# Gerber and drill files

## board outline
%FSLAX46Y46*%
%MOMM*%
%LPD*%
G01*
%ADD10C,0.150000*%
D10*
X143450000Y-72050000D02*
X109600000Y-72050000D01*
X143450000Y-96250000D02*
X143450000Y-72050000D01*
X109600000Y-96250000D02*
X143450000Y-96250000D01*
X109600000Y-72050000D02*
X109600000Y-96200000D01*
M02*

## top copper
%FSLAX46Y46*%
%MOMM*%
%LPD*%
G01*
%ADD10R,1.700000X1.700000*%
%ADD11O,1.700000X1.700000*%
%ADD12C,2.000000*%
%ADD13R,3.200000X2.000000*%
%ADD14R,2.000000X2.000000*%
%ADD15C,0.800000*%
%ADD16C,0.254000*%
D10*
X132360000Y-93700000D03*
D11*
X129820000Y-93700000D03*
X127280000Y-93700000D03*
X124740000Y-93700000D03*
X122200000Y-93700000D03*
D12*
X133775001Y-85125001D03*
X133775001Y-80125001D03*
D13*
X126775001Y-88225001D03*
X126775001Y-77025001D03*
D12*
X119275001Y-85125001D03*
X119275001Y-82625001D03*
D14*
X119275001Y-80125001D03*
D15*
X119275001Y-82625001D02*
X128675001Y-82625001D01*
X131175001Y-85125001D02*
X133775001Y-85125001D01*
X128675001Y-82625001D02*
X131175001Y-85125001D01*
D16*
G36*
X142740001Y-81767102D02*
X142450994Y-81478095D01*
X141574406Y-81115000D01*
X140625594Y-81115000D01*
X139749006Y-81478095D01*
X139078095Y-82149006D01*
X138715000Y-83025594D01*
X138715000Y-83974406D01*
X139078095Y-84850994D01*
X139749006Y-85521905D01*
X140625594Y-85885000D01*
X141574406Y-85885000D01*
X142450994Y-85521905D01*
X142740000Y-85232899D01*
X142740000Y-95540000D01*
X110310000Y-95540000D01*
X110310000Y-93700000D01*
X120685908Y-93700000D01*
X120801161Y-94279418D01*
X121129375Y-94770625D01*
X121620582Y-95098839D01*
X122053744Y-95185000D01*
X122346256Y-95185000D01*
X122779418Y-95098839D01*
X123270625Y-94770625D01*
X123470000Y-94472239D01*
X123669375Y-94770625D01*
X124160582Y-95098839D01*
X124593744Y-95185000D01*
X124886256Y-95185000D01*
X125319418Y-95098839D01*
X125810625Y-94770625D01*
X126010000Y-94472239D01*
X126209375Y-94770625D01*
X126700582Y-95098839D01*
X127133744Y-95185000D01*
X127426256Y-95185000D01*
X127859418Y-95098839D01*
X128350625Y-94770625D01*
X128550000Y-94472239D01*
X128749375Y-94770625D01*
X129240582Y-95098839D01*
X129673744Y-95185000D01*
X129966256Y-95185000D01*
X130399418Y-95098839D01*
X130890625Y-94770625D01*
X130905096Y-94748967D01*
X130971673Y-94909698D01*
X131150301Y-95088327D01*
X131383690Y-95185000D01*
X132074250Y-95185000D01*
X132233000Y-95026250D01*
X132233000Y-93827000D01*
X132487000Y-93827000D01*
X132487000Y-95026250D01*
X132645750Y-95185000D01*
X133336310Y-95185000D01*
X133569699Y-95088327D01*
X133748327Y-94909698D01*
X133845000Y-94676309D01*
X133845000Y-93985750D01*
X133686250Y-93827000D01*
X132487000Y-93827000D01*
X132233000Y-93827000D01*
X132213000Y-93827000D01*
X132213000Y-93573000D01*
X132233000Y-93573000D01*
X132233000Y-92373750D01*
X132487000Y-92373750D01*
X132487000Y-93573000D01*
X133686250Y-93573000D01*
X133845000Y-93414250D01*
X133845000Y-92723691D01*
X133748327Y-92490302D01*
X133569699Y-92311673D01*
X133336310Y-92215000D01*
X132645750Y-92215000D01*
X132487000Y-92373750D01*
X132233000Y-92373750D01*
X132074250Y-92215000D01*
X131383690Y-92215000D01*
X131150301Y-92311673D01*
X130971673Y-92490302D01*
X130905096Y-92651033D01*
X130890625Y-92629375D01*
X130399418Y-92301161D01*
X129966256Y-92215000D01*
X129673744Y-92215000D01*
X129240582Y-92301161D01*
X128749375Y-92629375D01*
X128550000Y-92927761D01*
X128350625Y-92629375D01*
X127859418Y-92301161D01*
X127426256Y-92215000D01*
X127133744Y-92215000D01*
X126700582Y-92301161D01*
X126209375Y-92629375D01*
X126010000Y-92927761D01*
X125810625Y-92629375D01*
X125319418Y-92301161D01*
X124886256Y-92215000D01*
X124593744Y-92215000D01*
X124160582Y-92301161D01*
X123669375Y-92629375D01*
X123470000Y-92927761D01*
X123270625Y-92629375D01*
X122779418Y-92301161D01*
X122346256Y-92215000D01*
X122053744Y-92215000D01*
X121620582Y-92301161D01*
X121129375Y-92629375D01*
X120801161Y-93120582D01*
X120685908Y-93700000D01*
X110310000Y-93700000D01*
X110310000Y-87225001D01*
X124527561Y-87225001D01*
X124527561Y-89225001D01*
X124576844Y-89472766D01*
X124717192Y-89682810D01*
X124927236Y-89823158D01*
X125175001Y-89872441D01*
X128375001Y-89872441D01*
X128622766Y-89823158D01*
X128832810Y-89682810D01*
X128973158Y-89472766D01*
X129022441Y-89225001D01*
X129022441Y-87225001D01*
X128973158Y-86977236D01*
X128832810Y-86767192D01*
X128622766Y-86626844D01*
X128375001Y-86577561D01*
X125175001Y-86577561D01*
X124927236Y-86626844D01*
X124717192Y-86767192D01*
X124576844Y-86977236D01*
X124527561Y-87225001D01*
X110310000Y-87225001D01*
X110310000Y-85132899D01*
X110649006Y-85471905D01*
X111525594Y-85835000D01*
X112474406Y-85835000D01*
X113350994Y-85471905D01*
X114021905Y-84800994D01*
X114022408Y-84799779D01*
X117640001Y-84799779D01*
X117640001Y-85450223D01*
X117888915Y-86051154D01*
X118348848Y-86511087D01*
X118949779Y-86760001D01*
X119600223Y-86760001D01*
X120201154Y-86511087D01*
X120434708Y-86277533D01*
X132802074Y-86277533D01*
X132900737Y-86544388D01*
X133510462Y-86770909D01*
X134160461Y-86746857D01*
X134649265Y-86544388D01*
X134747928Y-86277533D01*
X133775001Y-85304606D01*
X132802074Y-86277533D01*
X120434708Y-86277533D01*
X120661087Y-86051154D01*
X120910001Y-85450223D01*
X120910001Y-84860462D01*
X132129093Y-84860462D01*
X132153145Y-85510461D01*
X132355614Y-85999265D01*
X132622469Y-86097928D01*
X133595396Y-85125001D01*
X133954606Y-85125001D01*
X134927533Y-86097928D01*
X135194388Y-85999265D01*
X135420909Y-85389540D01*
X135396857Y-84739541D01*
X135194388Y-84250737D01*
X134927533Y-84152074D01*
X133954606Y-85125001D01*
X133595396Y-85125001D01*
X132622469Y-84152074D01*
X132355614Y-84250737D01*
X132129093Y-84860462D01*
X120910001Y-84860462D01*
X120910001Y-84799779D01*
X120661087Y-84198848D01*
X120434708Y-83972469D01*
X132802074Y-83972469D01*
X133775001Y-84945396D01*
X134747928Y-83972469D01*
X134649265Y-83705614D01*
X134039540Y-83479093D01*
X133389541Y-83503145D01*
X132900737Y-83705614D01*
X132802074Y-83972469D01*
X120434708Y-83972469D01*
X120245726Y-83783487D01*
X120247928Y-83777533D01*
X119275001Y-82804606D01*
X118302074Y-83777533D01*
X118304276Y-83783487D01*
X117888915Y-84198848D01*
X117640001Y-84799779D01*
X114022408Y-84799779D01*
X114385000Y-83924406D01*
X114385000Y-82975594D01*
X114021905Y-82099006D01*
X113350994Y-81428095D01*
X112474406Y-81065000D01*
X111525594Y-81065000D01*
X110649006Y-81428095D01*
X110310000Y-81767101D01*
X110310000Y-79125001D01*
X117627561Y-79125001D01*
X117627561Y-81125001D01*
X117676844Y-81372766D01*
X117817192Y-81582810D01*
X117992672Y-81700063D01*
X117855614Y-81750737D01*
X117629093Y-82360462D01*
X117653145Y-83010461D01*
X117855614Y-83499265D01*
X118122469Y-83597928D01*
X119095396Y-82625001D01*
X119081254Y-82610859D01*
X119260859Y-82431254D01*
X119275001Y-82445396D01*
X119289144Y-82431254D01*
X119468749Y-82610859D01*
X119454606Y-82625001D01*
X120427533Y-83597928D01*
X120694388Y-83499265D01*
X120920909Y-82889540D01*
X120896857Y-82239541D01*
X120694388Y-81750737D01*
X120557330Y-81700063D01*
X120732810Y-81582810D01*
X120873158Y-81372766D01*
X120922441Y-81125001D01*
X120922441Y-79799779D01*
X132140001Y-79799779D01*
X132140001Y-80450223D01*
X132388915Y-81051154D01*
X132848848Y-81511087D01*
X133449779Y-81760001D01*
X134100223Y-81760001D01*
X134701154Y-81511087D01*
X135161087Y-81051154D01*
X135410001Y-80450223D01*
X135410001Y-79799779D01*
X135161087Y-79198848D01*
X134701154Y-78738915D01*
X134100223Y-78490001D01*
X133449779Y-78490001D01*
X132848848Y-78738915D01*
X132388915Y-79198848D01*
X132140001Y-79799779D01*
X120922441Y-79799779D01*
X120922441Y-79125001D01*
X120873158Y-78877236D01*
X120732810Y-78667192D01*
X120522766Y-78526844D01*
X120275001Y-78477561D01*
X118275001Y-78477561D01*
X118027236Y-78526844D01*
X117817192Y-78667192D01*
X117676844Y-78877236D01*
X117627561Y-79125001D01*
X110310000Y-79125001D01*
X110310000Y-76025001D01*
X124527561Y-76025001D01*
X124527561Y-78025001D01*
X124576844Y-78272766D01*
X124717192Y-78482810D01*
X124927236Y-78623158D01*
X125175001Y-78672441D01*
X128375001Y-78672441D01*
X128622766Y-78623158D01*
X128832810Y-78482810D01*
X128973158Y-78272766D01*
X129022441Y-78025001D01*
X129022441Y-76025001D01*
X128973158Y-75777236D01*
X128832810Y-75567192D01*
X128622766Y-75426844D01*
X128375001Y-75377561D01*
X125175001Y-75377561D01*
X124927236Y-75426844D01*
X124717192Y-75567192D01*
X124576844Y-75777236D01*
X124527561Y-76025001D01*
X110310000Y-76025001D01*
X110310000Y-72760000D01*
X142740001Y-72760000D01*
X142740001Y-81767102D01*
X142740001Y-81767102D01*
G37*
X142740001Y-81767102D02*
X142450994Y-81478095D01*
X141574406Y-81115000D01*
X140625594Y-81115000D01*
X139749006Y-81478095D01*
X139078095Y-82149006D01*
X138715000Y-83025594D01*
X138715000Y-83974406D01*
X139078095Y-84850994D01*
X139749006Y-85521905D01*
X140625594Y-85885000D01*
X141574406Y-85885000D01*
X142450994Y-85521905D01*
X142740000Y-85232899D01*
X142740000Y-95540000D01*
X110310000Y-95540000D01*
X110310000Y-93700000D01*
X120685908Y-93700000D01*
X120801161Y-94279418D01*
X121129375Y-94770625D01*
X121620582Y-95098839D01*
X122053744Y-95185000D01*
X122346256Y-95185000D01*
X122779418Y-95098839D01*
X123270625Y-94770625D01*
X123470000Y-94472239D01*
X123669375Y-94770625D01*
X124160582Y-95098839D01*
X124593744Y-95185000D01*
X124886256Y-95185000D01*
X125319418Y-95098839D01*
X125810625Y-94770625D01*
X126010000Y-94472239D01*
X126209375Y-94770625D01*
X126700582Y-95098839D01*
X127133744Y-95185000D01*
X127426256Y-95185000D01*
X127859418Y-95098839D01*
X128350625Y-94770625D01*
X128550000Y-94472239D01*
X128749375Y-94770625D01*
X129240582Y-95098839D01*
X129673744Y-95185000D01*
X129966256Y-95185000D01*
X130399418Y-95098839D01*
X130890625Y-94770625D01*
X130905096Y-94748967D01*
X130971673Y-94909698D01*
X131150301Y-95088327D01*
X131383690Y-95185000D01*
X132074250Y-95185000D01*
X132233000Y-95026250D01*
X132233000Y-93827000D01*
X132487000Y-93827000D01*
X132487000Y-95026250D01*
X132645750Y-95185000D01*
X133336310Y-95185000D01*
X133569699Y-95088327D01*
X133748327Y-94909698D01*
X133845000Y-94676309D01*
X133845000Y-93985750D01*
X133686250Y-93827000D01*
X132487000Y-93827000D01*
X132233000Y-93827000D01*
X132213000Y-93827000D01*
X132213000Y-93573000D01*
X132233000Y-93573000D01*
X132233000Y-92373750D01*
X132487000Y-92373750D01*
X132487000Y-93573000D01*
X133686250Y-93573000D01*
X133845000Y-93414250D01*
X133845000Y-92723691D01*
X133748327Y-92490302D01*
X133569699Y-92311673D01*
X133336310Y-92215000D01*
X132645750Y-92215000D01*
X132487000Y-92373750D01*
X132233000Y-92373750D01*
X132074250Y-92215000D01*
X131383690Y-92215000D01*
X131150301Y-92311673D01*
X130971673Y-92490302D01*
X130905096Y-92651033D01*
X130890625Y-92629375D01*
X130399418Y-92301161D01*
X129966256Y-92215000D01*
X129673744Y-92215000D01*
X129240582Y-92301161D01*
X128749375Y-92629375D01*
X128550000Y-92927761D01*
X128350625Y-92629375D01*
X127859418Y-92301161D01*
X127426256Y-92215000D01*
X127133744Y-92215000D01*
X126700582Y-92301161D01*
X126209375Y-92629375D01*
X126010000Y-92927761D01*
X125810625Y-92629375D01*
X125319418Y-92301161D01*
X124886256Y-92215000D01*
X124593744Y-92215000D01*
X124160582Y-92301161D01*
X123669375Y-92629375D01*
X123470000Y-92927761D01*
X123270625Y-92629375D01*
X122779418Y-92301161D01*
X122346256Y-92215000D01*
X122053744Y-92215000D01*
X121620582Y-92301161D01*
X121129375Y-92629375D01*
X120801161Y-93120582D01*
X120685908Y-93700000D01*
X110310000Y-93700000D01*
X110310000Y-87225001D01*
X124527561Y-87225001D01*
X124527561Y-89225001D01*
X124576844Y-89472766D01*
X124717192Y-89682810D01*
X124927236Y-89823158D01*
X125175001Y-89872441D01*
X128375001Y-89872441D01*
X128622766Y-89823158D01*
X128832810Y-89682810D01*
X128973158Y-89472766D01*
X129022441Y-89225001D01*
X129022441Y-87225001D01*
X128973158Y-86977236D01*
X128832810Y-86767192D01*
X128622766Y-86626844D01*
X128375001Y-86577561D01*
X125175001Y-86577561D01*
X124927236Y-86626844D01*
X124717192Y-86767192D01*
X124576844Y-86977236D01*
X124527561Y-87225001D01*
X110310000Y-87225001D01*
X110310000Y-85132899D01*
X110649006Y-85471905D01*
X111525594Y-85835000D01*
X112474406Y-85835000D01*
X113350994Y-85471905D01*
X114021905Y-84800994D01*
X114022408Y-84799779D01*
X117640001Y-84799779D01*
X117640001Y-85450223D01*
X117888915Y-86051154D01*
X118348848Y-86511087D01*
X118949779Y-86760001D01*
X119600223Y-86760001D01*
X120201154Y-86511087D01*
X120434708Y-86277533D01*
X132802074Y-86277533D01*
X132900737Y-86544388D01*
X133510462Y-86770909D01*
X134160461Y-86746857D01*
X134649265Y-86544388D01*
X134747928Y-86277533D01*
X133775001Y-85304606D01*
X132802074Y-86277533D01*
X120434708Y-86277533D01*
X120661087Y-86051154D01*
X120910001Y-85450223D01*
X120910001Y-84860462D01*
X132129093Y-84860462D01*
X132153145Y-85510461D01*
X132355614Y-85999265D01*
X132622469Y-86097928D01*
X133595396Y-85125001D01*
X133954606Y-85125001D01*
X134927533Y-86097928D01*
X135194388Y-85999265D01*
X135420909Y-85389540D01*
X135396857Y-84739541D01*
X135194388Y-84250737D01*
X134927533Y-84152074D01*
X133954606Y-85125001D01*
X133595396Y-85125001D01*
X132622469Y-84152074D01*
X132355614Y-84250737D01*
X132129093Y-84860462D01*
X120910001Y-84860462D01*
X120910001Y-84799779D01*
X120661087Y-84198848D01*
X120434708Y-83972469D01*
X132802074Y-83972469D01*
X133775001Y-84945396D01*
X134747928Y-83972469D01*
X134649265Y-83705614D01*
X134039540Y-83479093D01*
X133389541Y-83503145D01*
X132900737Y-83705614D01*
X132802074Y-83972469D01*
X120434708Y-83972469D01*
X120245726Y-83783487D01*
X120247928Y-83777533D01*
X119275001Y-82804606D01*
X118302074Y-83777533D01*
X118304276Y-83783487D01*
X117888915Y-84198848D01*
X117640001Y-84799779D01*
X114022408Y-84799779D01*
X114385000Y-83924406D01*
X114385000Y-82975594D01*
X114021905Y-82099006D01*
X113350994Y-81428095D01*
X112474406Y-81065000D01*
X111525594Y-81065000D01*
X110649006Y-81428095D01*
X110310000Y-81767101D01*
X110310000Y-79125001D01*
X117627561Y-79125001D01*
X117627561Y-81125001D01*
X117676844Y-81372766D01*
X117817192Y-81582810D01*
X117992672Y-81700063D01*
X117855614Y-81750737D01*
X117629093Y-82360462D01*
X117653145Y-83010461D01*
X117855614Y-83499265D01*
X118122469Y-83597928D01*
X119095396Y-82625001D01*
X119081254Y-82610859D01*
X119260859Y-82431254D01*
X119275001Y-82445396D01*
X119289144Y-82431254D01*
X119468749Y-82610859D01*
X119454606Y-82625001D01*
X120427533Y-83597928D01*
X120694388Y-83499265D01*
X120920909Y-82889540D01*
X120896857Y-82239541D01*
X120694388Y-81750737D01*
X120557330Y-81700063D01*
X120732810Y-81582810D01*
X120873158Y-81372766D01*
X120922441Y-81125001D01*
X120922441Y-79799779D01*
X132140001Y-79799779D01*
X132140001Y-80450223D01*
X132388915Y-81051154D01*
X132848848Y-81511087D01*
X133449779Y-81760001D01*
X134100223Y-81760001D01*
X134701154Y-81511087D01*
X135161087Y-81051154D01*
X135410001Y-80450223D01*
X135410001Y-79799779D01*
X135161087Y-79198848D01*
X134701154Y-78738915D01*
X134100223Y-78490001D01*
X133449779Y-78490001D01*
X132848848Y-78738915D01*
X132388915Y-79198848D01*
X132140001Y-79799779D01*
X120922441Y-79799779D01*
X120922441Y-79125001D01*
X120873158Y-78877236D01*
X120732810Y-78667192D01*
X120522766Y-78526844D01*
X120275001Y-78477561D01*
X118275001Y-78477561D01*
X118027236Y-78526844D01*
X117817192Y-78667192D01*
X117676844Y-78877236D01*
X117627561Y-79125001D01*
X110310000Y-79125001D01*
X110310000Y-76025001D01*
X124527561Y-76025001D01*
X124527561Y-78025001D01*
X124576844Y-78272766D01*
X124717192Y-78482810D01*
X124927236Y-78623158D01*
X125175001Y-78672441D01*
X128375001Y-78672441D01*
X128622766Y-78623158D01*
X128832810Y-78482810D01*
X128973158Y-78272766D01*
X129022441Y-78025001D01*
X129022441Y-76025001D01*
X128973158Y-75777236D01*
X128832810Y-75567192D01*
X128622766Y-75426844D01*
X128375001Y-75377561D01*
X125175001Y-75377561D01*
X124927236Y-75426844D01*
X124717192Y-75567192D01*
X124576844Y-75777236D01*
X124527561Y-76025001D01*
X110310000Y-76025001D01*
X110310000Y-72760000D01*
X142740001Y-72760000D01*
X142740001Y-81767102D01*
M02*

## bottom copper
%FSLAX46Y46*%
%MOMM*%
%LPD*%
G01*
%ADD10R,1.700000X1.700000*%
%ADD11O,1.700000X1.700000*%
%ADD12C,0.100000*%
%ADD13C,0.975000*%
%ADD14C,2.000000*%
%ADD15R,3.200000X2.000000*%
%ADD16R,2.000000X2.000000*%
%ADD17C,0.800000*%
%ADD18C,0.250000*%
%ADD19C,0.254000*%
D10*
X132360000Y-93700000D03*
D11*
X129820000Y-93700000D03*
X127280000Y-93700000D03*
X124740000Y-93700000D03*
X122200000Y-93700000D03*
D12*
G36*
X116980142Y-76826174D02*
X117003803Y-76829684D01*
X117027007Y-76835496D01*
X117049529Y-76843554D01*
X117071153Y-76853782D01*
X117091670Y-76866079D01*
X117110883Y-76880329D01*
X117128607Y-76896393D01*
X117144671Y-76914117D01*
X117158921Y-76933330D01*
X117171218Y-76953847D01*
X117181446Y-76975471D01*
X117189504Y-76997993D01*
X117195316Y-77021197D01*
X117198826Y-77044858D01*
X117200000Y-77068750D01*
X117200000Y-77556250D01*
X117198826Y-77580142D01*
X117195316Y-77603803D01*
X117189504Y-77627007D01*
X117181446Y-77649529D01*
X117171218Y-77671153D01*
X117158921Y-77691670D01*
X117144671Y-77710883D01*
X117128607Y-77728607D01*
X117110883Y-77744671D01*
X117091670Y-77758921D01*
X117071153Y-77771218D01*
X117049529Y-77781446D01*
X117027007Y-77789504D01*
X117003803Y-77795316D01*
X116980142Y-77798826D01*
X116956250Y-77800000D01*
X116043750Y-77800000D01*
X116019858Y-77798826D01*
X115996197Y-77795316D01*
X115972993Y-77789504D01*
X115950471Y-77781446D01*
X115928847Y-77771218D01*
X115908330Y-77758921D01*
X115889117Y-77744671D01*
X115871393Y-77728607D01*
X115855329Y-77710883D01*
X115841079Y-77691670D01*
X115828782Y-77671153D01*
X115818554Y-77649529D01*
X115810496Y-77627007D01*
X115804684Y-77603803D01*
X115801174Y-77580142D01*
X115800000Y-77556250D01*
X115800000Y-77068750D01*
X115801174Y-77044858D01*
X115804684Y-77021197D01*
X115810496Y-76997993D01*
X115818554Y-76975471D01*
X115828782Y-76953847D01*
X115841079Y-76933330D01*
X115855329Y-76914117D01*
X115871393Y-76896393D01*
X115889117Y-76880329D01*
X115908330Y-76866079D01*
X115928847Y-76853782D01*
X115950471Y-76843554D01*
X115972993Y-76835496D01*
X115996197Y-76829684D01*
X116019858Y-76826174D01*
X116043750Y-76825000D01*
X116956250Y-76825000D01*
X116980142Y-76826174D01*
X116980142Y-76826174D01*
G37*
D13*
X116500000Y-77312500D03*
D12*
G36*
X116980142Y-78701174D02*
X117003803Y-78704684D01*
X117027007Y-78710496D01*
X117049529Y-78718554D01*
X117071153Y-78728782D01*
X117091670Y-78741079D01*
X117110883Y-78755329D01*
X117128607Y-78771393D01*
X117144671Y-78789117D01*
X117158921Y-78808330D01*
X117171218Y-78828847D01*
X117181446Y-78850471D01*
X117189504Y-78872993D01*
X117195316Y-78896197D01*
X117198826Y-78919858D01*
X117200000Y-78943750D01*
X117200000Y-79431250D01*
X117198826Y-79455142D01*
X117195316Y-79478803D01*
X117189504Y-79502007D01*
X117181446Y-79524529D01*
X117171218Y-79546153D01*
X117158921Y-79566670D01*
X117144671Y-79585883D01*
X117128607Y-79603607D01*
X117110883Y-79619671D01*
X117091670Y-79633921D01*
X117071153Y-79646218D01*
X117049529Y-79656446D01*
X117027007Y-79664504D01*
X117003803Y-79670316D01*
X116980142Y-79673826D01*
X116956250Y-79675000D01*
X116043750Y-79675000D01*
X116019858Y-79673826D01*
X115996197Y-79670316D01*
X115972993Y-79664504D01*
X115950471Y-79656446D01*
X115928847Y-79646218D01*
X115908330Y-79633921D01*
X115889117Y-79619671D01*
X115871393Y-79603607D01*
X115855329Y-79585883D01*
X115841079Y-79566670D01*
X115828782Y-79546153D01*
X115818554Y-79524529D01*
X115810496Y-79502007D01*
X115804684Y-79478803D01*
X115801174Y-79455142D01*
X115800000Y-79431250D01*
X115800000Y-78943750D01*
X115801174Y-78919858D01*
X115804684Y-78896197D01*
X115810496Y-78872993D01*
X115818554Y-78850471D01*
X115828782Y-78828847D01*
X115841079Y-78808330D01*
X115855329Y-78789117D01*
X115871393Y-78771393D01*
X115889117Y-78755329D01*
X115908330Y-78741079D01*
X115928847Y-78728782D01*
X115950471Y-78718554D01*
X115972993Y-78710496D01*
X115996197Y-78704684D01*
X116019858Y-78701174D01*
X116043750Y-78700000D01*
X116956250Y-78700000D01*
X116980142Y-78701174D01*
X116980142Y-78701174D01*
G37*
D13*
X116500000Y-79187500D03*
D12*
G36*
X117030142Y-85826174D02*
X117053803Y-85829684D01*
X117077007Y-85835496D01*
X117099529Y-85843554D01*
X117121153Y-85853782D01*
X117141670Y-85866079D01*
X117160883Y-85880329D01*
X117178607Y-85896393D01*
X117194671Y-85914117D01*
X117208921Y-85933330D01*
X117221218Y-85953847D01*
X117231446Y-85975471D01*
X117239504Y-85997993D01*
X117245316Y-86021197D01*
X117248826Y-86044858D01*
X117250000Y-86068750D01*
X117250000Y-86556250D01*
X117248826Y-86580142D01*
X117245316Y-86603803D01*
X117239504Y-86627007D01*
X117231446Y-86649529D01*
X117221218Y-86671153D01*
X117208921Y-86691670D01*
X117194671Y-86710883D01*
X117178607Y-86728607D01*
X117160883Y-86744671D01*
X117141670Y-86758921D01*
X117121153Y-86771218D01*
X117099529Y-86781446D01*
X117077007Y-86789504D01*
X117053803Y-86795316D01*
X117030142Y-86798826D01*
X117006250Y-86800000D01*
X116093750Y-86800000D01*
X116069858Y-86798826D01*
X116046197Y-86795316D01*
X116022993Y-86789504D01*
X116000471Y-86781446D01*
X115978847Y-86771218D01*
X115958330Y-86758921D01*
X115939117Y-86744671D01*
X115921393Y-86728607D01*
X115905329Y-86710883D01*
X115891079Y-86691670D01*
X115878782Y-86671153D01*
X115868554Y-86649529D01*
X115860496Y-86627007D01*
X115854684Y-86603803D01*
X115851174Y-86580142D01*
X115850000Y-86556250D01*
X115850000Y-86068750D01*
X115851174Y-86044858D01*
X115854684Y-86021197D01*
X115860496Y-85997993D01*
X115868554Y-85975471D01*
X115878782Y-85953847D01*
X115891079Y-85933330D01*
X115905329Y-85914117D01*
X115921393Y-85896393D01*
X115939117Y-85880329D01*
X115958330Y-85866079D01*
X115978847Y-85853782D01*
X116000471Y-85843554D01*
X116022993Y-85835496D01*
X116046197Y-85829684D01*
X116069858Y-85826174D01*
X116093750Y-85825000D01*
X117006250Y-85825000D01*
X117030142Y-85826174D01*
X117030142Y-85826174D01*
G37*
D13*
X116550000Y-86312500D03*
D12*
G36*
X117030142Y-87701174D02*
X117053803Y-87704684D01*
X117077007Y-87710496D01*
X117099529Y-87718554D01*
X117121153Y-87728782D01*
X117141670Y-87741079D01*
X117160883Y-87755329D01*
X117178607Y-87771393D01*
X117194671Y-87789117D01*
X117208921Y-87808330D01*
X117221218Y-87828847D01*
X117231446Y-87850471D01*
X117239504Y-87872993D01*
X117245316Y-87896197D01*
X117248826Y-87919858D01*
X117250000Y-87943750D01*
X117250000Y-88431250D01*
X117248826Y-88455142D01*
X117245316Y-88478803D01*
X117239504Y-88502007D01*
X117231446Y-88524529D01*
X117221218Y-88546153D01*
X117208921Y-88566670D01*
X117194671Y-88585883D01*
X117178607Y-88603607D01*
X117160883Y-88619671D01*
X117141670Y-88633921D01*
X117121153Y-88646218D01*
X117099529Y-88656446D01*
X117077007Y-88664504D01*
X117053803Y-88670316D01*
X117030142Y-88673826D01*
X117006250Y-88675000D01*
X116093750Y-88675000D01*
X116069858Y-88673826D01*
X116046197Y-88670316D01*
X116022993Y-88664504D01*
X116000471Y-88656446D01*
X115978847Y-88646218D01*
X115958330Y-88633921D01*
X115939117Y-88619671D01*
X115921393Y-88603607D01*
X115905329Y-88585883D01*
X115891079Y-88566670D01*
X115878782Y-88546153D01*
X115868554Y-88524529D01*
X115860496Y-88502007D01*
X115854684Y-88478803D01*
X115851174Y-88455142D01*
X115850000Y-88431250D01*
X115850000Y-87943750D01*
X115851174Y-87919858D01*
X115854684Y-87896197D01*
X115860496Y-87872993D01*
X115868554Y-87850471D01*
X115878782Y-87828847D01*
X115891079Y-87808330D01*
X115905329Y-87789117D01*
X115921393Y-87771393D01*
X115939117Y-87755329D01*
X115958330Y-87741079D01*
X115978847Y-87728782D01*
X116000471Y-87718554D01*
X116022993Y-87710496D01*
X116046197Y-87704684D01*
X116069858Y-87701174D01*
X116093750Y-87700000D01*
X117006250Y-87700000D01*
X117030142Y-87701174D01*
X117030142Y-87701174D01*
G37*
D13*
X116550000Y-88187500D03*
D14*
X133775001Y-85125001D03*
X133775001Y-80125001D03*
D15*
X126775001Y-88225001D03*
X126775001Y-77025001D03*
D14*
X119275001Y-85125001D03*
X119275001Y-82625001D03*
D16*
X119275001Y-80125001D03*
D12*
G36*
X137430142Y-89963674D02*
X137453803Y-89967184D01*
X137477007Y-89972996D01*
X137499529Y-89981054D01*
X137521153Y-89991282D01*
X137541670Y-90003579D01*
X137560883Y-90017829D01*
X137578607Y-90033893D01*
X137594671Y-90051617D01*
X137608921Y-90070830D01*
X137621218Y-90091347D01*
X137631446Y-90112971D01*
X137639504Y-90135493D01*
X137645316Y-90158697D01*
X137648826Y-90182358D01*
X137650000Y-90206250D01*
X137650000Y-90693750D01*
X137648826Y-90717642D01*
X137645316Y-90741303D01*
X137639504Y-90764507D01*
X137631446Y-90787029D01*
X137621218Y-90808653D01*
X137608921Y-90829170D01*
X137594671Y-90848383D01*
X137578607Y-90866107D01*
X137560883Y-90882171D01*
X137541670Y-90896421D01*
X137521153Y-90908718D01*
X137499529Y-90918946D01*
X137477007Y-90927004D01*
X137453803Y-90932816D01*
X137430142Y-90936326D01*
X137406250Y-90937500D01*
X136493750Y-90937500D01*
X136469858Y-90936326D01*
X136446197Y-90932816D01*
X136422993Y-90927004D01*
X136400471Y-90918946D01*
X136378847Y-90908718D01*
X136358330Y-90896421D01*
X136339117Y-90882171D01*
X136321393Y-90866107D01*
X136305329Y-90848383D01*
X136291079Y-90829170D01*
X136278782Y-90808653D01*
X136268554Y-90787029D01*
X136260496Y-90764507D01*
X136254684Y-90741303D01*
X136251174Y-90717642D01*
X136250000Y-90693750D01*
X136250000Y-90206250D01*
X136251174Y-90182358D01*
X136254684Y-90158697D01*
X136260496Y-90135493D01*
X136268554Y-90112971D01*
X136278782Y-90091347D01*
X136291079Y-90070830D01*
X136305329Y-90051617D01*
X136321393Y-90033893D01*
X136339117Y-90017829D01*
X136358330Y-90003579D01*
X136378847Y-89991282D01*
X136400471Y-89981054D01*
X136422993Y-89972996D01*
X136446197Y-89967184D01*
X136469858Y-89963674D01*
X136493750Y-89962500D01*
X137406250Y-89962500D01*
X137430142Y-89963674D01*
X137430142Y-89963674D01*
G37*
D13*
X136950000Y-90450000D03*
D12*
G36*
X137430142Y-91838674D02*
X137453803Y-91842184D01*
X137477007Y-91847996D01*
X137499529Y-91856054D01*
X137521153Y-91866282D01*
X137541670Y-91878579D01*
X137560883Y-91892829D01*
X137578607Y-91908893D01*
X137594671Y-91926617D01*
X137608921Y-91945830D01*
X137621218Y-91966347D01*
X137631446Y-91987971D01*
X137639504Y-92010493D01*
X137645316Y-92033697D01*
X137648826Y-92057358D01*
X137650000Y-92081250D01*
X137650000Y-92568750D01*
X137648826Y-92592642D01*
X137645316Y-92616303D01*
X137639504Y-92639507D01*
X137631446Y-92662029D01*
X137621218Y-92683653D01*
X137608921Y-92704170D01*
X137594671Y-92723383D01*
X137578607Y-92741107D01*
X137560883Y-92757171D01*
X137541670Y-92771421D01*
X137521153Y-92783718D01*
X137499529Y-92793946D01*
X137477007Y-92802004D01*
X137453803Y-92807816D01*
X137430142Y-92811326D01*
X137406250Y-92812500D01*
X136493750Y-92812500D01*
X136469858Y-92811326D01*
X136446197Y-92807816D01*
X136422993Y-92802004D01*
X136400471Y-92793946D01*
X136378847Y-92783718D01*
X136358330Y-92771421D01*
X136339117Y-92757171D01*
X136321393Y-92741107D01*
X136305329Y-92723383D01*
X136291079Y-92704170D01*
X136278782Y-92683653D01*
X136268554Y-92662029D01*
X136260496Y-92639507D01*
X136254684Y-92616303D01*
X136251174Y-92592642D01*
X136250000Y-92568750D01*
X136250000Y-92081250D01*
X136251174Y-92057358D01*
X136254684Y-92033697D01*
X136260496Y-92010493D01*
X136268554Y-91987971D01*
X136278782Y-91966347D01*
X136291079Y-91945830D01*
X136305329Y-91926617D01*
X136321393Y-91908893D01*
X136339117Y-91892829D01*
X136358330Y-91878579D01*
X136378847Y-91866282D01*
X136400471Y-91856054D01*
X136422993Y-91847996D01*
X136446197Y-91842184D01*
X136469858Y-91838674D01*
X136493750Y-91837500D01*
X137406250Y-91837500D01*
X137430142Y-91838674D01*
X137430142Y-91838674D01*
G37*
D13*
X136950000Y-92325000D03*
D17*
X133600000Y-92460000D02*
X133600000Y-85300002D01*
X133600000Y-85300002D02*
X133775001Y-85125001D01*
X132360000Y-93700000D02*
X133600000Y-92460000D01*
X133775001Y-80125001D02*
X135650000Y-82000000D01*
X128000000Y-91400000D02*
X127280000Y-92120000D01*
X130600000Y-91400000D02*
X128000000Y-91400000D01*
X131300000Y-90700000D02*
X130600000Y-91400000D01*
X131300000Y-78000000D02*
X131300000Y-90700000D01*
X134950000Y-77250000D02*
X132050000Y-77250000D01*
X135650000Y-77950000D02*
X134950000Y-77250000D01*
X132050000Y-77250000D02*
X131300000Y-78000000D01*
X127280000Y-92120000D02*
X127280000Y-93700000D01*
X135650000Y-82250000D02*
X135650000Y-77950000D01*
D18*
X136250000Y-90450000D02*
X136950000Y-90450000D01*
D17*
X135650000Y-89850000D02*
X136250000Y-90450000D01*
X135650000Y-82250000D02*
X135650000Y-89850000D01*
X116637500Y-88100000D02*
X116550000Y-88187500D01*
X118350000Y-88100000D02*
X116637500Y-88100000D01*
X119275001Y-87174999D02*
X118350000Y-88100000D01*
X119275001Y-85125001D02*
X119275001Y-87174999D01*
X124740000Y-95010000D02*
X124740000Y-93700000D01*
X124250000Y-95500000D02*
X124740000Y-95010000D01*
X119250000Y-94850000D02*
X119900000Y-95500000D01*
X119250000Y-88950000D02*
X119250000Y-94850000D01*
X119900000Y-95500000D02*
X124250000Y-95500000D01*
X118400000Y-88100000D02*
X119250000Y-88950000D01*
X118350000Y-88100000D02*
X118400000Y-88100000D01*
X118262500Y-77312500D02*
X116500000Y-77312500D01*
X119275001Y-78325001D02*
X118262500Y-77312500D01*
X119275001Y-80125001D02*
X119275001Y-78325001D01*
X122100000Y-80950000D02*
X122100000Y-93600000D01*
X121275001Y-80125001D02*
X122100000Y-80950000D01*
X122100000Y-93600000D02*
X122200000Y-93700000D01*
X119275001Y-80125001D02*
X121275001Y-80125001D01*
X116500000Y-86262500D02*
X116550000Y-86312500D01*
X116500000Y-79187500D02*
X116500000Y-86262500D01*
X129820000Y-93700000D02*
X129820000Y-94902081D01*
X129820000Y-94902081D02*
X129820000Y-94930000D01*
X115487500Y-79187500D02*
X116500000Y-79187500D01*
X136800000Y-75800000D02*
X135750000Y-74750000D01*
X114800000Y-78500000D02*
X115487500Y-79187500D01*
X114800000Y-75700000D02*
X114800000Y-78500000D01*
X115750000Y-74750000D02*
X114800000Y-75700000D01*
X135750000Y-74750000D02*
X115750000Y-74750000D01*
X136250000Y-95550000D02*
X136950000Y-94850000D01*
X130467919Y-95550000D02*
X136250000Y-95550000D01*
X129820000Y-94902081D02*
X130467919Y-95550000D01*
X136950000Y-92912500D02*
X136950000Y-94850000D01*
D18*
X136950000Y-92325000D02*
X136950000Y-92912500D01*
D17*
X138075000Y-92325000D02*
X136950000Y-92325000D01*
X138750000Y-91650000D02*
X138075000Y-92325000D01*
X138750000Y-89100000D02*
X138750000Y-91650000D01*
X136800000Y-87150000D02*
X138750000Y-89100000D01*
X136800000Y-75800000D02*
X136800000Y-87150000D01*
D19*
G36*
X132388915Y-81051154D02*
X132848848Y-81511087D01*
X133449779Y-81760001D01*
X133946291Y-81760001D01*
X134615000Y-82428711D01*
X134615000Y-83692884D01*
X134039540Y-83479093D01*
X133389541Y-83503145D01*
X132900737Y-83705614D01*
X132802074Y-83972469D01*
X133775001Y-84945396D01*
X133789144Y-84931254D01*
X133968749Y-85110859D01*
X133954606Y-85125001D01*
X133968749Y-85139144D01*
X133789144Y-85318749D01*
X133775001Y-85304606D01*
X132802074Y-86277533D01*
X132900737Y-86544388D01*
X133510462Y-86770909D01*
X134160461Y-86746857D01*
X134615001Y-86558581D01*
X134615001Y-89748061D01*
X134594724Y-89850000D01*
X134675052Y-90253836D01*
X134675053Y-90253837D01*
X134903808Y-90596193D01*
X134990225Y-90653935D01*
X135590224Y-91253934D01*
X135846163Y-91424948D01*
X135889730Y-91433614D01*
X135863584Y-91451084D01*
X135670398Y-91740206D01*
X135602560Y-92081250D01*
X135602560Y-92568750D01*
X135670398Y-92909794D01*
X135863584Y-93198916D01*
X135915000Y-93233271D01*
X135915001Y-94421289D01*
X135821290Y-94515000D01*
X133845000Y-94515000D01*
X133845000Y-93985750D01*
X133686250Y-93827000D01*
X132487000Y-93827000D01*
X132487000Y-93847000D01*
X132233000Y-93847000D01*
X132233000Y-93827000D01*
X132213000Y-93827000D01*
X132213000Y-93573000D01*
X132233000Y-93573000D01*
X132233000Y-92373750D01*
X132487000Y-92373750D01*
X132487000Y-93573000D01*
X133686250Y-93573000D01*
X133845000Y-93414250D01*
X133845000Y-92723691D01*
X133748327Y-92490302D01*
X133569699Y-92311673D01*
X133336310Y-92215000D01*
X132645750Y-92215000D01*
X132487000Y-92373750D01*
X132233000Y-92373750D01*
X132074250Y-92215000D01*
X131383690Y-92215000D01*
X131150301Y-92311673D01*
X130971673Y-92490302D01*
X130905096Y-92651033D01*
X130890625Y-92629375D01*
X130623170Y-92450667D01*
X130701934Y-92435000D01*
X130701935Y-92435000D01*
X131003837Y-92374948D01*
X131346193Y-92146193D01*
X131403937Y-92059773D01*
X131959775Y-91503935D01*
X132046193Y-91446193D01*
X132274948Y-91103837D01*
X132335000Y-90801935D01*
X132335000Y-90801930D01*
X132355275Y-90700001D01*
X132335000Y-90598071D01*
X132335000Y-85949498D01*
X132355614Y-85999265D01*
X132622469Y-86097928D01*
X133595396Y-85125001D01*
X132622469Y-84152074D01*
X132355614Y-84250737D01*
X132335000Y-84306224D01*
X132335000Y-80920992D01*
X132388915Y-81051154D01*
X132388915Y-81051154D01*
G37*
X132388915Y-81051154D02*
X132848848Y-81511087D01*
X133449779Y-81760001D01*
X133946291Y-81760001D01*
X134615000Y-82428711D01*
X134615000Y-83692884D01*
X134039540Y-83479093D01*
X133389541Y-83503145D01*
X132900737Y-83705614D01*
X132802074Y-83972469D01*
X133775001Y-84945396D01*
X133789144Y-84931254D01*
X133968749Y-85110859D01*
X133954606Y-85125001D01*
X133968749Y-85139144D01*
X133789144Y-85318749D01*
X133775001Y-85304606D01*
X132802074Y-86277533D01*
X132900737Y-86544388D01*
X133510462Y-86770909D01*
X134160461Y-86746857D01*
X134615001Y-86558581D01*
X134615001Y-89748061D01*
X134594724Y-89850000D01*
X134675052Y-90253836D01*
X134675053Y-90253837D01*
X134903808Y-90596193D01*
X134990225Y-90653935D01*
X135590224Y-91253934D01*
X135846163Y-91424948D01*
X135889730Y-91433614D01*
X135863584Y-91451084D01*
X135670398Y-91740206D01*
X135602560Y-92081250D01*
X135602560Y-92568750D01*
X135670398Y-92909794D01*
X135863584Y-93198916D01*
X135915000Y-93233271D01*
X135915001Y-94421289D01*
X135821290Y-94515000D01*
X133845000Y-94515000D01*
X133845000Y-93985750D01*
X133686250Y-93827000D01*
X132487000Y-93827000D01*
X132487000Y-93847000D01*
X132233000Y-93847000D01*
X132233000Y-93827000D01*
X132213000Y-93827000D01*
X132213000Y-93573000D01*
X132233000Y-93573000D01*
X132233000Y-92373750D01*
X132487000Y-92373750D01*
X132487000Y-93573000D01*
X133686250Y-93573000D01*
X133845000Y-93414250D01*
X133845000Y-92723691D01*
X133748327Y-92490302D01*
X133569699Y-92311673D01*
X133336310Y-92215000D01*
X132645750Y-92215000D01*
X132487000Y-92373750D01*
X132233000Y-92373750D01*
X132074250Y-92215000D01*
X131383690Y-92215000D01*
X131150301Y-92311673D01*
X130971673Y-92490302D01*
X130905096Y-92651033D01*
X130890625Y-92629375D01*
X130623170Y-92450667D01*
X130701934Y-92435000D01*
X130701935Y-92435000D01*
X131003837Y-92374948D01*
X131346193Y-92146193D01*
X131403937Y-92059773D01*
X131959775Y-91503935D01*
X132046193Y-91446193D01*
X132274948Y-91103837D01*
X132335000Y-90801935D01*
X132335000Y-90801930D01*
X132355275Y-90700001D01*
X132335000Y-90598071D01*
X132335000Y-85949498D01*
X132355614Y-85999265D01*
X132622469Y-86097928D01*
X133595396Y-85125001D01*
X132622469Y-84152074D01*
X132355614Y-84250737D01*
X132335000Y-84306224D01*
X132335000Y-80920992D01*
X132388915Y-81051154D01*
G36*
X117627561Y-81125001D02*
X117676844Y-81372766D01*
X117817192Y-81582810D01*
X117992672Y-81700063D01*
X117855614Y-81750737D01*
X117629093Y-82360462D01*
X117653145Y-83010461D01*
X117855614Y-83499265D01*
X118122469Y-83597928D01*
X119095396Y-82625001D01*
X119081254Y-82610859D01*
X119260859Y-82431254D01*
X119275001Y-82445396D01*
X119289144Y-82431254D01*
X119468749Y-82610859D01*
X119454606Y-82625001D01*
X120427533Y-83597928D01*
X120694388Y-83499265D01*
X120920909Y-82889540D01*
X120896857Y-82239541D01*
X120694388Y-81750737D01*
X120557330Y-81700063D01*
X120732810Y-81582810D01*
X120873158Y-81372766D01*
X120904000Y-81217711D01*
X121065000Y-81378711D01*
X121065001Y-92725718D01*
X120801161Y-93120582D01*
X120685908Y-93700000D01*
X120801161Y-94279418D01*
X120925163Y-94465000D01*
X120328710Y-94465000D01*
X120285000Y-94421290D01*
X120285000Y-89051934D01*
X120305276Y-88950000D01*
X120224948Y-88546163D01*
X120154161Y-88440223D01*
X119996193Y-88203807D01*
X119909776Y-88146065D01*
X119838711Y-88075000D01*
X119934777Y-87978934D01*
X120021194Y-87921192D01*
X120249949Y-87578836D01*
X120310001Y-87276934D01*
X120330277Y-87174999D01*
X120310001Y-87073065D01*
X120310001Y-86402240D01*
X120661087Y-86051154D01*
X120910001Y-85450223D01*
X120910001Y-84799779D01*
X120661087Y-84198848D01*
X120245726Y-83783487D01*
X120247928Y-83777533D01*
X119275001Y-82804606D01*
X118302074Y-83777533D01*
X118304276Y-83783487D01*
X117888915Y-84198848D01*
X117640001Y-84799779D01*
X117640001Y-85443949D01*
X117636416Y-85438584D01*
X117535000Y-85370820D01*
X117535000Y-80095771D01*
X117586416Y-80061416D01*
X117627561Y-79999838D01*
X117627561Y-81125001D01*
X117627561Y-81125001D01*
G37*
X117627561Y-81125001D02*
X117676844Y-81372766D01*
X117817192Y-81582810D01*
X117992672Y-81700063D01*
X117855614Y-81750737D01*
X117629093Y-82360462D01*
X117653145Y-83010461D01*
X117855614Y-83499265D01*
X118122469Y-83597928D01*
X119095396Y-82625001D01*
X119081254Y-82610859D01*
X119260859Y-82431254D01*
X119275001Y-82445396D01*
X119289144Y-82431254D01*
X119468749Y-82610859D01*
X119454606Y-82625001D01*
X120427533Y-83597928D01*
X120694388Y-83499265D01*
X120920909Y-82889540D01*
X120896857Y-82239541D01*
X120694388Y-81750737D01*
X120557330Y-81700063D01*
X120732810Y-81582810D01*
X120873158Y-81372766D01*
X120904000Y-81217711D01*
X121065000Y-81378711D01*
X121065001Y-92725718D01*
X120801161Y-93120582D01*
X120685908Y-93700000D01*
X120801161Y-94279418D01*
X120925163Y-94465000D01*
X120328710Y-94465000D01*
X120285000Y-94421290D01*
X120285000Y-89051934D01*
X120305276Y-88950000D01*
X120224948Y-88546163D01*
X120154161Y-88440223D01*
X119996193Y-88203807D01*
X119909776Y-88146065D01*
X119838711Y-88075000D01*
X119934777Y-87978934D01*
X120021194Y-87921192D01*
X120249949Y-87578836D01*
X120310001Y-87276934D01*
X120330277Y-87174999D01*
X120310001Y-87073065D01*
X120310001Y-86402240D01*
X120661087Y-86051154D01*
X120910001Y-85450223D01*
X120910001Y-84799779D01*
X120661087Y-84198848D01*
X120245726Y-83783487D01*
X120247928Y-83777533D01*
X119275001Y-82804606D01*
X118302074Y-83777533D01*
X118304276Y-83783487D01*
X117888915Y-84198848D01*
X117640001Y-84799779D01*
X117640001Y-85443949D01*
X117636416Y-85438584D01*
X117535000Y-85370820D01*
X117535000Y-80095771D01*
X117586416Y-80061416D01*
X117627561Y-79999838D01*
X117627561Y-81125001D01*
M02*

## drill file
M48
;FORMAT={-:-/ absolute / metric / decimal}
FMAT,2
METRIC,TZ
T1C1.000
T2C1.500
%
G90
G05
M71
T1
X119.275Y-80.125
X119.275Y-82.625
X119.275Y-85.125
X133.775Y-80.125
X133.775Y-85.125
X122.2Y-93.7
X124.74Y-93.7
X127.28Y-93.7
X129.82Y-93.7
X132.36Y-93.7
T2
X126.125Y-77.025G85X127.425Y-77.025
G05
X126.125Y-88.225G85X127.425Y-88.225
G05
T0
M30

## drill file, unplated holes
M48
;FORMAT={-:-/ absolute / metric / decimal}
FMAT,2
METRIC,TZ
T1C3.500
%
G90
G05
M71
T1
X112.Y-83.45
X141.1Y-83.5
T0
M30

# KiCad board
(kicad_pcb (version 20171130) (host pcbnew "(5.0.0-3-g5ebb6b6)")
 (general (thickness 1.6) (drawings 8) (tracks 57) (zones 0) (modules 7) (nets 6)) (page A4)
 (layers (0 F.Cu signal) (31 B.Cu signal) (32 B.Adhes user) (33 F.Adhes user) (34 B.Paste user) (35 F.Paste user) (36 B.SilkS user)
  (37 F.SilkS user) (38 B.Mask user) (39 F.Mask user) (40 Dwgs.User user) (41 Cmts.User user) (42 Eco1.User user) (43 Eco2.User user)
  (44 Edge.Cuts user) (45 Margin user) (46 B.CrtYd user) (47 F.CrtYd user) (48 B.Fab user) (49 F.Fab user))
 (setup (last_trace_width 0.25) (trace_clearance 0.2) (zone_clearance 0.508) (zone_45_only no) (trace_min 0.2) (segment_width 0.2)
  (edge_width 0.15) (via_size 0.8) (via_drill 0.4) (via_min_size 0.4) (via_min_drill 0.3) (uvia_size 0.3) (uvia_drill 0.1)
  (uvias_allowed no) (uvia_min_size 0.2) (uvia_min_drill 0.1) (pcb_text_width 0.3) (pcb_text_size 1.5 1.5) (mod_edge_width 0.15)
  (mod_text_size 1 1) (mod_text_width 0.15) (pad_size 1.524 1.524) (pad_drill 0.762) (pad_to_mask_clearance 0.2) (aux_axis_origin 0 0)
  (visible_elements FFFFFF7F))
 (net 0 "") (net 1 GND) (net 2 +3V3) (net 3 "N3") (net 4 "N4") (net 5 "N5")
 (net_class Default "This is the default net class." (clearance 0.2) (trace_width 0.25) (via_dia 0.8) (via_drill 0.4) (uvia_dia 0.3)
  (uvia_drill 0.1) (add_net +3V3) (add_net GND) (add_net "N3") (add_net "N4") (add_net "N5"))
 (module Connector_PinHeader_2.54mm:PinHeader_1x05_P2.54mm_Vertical (layer F.Cu) (at 132.36 93.7 270)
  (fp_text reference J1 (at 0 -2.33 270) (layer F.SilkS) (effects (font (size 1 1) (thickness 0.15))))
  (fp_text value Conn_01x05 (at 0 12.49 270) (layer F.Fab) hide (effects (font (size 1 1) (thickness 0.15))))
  (pad 1 thru_hole rect (at 0 0 270) (size 1.7 1.7) (drill 1) (layers *.Cu *.Mask) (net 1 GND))
  (pad 2 thru_hole oval (at 0 2.54 270) (size 1.7 1.7) (drill 1) (layers *.Cu *.Mask) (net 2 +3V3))
  (pad 3 thru_hole oval (at 0 5.08 270) (size 1.7 1.7) (drill 1) (layers *.Cu *.Mask) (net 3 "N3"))
  (pad 4 thru_hole oval (at 0 7.62 270) (size 1.7 1.7) (drill 1) (layers *.Cu *.Mask) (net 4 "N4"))
  (pad 5 thru_hole oval (at 0 10.16 270) (size 1.7 1.7) (drill 1) (layers *.Cu *.Mask) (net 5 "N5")))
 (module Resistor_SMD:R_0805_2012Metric (layer B.Cu) (at 116.5 78.25 270)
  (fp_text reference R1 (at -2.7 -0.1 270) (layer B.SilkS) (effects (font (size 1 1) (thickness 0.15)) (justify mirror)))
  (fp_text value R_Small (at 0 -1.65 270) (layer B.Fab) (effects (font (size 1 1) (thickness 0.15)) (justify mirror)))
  (pad 1 smd roundrect (at -0.9375 0 270) (size 0.975 1.4) (layers B.Cu B.Paste B.Mask) (roundrect_rratio 0.25) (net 5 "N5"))
  (pad 2 smd roundrect (at 0.9375 0 270) (size 0.975 1.4) (layers B.Cu B.Paste B.Mask) (roundrect_rratio 0.25) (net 2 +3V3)))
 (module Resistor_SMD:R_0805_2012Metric (layer B.Cu) (at 116.55 87.25 90)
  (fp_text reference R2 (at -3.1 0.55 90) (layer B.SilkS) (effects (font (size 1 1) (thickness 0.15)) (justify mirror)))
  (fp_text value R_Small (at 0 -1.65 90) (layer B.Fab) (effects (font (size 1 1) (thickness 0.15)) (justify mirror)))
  (pad 2 smd roundrect (at 0.9375 0 90) (size 0.975 1.4) (layers B.Cu B.Paste B.Mask) (roundrect_rratio 0.25) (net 2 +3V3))
  (pad 1 smd roundrect (at -0.9375 0 90) (size 0.975 1.4) (layers B.Cu B.Paste B.Mask) (roundrect_rratio 0.25) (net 4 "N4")))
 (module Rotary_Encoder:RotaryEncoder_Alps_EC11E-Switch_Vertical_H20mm (layer F.Cu) (at 119.275001 80.125001)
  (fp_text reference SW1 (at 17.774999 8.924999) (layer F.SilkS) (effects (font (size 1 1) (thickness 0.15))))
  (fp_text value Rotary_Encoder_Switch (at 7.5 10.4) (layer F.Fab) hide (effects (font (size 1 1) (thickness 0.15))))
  (pad S1 thru_hole circle (at 14.5 5) (size 2 2) (drill 1) (layers *.Cu *.Mask) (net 1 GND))
  (pad S2 thru_hole circle (at 14.5 0) (size 2 2) (drill 1) (layers *.Cu *.Mask) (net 3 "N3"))
  (pad MP thru_hole rect (at 7.5 8.1) (size 3.2 2) (drill oval 2.8 1.5) (layers *.Cu *.Mask))
  (pad MP thru_hole rect (at 7.5 -3.1) (size 3.2 2) (drill oval 2.8 1.5) (layers *.Cu *.Mask))
  (pad B thru_hole circle (at 0 5) (size 2 2) (drill 1) (layers *.Cu *.Mask) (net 4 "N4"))
  (pad C thru_hole circle (at 0 2.5) (size 2 2) (drill 1) (layers *.Cu *.Mask) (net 1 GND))
  (pad A thru_hole rect (at 0 0) (size 2 2) (drill 1) (layers *.Cu *.Mask) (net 5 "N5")))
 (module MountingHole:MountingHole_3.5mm (layer F.Cu) (at 112 83.45)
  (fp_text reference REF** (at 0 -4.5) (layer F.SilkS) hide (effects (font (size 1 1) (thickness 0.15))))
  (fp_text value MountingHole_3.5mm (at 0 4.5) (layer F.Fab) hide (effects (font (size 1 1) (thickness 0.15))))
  (pad 1 np_thru_hole circle (at 0 0) (size 3.5 3.5) (drill 3.5) (layers *.Cu *.Mask)))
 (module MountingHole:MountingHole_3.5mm (layer F.Cu) (at 141.1 83.5)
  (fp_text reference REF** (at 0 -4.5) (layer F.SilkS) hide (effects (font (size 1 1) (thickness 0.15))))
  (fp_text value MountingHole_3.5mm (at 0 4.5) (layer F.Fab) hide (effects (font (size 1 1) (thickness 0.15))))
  (pad 1 np_thru_hole circle (at 0 0) (size 3.5 3.5) (drill 3.5) (layers *.Cu *.Mask)))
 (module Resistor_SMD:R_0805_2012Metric (layer B.Cu) (at 136.95 91.3875 270)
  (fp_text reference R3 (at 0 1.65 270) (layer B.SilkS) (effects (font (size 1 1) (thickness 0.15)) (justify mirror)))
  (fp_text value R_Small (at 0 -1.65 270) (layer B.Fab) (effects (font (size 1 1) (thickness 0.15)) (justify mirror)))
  (pad 1 smd roundrect (at -0.9375 0 270) (size 0.975 1.4) (layers B.Cu B.Paste B.Mask) (roundrect_rratio 0.25) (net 3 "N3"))
  (pad 2 smd roundrect (at 0.9375 0 270) (size 0.975 1.4) (layers B.Cu B.Paste B.Mask) (roundrect_rratio 0.25) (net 2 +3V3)))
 (gr_line (start 143.45 72.05) (end 109.6 72.05) (layer Edge.Cuts) (width 0.15))
 (gr_line (start 143.45 96.25) (end 143.45 72.05) (layer Edge.Cuts) (width 0.15))
 (gr_line (start 109.6 96.25) (end 143.45 96.25) (layer Edge.Cuts) (width 0.15))
 (gr_line (start 109.6 72.05) (end 109.6 96.2) (layer Edge.Cuts) (width 0.15))
 (segment (start 119.275001 82.625001) (end 128.675001 82.625001) (width 0.8) (layer F.Cu) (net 1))
 (segment (start 131.175001 85.125001) (end 133.775001 85.125001) (width 0.8) (layer F.Cu) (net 1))
 (segment (start 128.675001 82.625001) (end 131.175001 85.125001) (width 0.8) (layer F.Cu) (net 1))
 (segment (start 133.6 92.46) (end 133.6 85.300002) (width 0.8) (layer B.Cu) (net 1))
 (segment (start 133.6 85.300002) (end 133.775001 85.125001) (width 0.8) (layer B.Cu) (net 1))
 (segment (start 132.36 93.7) (end 133.6 92.46) (width 0.8) (layer B.Cu) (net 1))
 (segment (start 133.775001 80.125001) (end 135.65 82) (width 0.8) (layer B.Cu) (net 3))
 (segment (start 128 91.4) (end 127.28 92.12) (width 0.8) (layer B.Cu) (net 3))
 (segment (start 130.6 91.4) (end 128 91.4) (width 0.8) (layer B.Cu) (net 3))
 (segment (start 131.3 90.7) (end 130.6 91.4) (width 0.8) (layer B.Cu) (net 3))
 (segment (start 131.3 78) (end 131.3 90.7) (width 0.8) (layer B.Cu) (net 3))
 (segment (start 134.95 77.25) (end 132.05 77.25) (width 0.8) (layer B.Cu) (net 3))
 (segment (start 135.65 77.95) (end 134.95 77.25) (width 0.8) (layer B.Cu) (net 3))
 (segment (start 132.05 77.25) (end 131.3 78) (width 0.8) (layer B.Cu) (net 3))
 (segment (start 127.28 92.12) (end 127.28 93.7) (width 0.8) (layer B.Cu) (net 3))
 (segment (start 135.65 82.25) (end 135.65 77.95) (width 0.8) (layer B.Cu) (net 3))
 (segment (start 136.25 90.45) (end 136.95 90.45) (width 0.25) (layer B.Cu) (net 3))
 (segment (start 135.65 89.85) (end 136.25 90.45) (width 0.8) (layer B.Cu) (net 3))
 (segment (start 135.65 82.25) (end 135.65 89.85) (width 0.8) (layer B.Cu) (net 3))
 (segment (start 116.6375 88.1) (end 116.55 88.1875) (width 0.8) (layer B.Cu) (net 4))
 (segment (start 118.35 88.1) (end 116.6375 88.1) (width 0.8) (layer B.Cu) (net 4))
 (segment (start 119.275001 87.174999) (end 118.35 88.1) (width 0.8) (layer B.Cu) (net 4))
 (segment (start 119.275001 85.125001) (end 119.275001 87.174999) (width 0.8) (layer B.Cu) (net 4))
 (segment (start 124.74 95.01) (end 124.74 93.7) (width 0.8) (layer B.Cu) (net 4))
 (segment (start 124.25 95.5) (end 124.74 95.01) (width 0.8) (layer B.Cu) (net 4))
 (segment (start 119.25 94.85) (end 119.9 95.5) (width 0.8) (layer B.Cu) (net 4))
 (segment (start 119.25 88.95) (end 119.25 94.85) (width 0.8) (layer B.Cu) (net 4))
 (segment (start 119.9 95.5) (end 124.25 95.5) (width 0.8) (layer B.Cu) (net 4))
 (segment (start 118.4 88.1) (end 119.25 88.95) (width 0.8) (layer B.Cu) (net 4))
 (segment (start 118.35 88.1) (end 118.4 88.1) (width 0.8) (layer B.Cu) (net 4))
 (segment (start 118.2625 77.3125) (end 116.5 77.3125) (width 0.8) (layer B.Cu) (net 5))
 (segment (start 119.275001 78.325001) (end 118.2625 77.3125) (width 0.8) (layer B.Cu) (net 5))
 (segment (start 119.275001 80.125001) (end 119.275001 78.325001) (width 0.8) (layer B.Cu) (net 5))
 (segment (start 122.1 80.95) (end 122.1 93.6) (width 0.8) (layer B.Cu) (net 5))
 (segment (start 121.275001 80.125001) (end 122.1 80.95) (width 0.8) (layer B.Cu) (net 5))
 (segment (start 122.1 93.6) (end 122.2 93.7) (width 0.8) (layer B.Cu) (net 5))
 (segment (start 119.275001 80.125001) (end 121.275001 80.125001) (width 0.8) (layer B.Cu) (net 5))
 (segment (start 116.5 86.2625) (end 116.55 86.3125) (width 0.8) (layer B.Cu) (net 2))
 (segment (start 116.5 79.1875) (end 116.5 86.2625) (width 0.8) (layer B.Cu) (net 2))
 (segment (start 129.82 93.7) (end 129.82 94.902081) (width 0.8) (layer B.Cu) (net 2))
 (segment (start 129.82 94.902081) (end 129.82 94.93) (width 0.8) (layer B.Cu) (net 2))
 (segment (start 115.4875 79.1875) (end 116.5 79.1875) (width 0.8) (layer B.Cu) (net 2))
 (segment (start 136.8 75.8) (end 135.75 74.75) (width 0.8) (layer B.Cu) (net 2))
 (segment (start 114.8 78.5) (end 115.4875 79.1875) (width 0.8) (layer B.Cu) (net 2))
 (segment (start 114.8 75.7) (end 114.8 78.5) (width 0.8) (layer B.Cu) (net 2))
 (segment (start 115.75 74.75) (end 114.8 75.7) (width 0.8) (layer B.Cu) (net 2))
 (segment (start 135.75 74.75) (end 115.75 74.75) (width 0.8) (layer B.Cu) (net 2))
 (segment (start 136.25 95.55) (end 136.95 94.85) (width 0.8) (layer B.Cu) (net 2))
 (segment (start 130.467919 95.55) (end 136.25 95.55) (width 0.8) (layer B.Cu) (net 2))
 (segment (start 129.82 94.902081) (end 130.467919 95.55) (width 0.8) (layer B.Cu) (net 2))
 (segment (start 136.95 92.9125) (end 136.95 94.85) (width 0.8) (layer B.Cu) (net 2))
 (segment (start 136.95 92.325) (end 136.95 92.9125) (width 0.25) (layer B.Cu) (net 2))
 (segment (start 138.075 92.325) (end 136.95 92.325) (width 0.8) (layer B.Cu) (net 2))
 (segment (start 138.75 91.65) (end 138.075 92.325) (width 0.8) (layer B.Cu) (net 2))
 (segment (start 138.75 89.1) (end 138.75 91.65) (width 0.8) (layer B.Cu) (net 2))
 (segment (start 136.8 87.15) (end 138.75 89.1) (width 0.8) (layer B.Cu) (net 2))
 (segment (start 136.8 75.8) (end 136.8 87.15) (width 0.8) (layer B.Cu) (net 2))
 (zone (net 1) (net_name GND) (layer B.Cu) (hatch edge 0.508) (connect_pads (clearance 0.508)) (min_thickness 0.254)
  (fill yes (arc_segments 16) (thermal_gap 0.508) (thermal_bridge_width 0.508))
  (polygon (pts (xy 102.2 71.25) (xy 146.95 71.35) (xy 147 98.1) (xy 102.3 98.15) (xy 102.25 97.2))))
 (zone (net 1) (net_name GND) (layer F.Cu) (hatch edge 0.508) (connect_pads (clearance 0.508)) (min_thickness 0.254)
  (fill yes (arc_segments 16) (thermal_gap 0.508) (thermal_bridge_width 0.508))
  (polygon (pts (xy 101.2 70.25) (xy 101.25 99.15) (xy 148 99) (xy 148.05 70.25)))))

